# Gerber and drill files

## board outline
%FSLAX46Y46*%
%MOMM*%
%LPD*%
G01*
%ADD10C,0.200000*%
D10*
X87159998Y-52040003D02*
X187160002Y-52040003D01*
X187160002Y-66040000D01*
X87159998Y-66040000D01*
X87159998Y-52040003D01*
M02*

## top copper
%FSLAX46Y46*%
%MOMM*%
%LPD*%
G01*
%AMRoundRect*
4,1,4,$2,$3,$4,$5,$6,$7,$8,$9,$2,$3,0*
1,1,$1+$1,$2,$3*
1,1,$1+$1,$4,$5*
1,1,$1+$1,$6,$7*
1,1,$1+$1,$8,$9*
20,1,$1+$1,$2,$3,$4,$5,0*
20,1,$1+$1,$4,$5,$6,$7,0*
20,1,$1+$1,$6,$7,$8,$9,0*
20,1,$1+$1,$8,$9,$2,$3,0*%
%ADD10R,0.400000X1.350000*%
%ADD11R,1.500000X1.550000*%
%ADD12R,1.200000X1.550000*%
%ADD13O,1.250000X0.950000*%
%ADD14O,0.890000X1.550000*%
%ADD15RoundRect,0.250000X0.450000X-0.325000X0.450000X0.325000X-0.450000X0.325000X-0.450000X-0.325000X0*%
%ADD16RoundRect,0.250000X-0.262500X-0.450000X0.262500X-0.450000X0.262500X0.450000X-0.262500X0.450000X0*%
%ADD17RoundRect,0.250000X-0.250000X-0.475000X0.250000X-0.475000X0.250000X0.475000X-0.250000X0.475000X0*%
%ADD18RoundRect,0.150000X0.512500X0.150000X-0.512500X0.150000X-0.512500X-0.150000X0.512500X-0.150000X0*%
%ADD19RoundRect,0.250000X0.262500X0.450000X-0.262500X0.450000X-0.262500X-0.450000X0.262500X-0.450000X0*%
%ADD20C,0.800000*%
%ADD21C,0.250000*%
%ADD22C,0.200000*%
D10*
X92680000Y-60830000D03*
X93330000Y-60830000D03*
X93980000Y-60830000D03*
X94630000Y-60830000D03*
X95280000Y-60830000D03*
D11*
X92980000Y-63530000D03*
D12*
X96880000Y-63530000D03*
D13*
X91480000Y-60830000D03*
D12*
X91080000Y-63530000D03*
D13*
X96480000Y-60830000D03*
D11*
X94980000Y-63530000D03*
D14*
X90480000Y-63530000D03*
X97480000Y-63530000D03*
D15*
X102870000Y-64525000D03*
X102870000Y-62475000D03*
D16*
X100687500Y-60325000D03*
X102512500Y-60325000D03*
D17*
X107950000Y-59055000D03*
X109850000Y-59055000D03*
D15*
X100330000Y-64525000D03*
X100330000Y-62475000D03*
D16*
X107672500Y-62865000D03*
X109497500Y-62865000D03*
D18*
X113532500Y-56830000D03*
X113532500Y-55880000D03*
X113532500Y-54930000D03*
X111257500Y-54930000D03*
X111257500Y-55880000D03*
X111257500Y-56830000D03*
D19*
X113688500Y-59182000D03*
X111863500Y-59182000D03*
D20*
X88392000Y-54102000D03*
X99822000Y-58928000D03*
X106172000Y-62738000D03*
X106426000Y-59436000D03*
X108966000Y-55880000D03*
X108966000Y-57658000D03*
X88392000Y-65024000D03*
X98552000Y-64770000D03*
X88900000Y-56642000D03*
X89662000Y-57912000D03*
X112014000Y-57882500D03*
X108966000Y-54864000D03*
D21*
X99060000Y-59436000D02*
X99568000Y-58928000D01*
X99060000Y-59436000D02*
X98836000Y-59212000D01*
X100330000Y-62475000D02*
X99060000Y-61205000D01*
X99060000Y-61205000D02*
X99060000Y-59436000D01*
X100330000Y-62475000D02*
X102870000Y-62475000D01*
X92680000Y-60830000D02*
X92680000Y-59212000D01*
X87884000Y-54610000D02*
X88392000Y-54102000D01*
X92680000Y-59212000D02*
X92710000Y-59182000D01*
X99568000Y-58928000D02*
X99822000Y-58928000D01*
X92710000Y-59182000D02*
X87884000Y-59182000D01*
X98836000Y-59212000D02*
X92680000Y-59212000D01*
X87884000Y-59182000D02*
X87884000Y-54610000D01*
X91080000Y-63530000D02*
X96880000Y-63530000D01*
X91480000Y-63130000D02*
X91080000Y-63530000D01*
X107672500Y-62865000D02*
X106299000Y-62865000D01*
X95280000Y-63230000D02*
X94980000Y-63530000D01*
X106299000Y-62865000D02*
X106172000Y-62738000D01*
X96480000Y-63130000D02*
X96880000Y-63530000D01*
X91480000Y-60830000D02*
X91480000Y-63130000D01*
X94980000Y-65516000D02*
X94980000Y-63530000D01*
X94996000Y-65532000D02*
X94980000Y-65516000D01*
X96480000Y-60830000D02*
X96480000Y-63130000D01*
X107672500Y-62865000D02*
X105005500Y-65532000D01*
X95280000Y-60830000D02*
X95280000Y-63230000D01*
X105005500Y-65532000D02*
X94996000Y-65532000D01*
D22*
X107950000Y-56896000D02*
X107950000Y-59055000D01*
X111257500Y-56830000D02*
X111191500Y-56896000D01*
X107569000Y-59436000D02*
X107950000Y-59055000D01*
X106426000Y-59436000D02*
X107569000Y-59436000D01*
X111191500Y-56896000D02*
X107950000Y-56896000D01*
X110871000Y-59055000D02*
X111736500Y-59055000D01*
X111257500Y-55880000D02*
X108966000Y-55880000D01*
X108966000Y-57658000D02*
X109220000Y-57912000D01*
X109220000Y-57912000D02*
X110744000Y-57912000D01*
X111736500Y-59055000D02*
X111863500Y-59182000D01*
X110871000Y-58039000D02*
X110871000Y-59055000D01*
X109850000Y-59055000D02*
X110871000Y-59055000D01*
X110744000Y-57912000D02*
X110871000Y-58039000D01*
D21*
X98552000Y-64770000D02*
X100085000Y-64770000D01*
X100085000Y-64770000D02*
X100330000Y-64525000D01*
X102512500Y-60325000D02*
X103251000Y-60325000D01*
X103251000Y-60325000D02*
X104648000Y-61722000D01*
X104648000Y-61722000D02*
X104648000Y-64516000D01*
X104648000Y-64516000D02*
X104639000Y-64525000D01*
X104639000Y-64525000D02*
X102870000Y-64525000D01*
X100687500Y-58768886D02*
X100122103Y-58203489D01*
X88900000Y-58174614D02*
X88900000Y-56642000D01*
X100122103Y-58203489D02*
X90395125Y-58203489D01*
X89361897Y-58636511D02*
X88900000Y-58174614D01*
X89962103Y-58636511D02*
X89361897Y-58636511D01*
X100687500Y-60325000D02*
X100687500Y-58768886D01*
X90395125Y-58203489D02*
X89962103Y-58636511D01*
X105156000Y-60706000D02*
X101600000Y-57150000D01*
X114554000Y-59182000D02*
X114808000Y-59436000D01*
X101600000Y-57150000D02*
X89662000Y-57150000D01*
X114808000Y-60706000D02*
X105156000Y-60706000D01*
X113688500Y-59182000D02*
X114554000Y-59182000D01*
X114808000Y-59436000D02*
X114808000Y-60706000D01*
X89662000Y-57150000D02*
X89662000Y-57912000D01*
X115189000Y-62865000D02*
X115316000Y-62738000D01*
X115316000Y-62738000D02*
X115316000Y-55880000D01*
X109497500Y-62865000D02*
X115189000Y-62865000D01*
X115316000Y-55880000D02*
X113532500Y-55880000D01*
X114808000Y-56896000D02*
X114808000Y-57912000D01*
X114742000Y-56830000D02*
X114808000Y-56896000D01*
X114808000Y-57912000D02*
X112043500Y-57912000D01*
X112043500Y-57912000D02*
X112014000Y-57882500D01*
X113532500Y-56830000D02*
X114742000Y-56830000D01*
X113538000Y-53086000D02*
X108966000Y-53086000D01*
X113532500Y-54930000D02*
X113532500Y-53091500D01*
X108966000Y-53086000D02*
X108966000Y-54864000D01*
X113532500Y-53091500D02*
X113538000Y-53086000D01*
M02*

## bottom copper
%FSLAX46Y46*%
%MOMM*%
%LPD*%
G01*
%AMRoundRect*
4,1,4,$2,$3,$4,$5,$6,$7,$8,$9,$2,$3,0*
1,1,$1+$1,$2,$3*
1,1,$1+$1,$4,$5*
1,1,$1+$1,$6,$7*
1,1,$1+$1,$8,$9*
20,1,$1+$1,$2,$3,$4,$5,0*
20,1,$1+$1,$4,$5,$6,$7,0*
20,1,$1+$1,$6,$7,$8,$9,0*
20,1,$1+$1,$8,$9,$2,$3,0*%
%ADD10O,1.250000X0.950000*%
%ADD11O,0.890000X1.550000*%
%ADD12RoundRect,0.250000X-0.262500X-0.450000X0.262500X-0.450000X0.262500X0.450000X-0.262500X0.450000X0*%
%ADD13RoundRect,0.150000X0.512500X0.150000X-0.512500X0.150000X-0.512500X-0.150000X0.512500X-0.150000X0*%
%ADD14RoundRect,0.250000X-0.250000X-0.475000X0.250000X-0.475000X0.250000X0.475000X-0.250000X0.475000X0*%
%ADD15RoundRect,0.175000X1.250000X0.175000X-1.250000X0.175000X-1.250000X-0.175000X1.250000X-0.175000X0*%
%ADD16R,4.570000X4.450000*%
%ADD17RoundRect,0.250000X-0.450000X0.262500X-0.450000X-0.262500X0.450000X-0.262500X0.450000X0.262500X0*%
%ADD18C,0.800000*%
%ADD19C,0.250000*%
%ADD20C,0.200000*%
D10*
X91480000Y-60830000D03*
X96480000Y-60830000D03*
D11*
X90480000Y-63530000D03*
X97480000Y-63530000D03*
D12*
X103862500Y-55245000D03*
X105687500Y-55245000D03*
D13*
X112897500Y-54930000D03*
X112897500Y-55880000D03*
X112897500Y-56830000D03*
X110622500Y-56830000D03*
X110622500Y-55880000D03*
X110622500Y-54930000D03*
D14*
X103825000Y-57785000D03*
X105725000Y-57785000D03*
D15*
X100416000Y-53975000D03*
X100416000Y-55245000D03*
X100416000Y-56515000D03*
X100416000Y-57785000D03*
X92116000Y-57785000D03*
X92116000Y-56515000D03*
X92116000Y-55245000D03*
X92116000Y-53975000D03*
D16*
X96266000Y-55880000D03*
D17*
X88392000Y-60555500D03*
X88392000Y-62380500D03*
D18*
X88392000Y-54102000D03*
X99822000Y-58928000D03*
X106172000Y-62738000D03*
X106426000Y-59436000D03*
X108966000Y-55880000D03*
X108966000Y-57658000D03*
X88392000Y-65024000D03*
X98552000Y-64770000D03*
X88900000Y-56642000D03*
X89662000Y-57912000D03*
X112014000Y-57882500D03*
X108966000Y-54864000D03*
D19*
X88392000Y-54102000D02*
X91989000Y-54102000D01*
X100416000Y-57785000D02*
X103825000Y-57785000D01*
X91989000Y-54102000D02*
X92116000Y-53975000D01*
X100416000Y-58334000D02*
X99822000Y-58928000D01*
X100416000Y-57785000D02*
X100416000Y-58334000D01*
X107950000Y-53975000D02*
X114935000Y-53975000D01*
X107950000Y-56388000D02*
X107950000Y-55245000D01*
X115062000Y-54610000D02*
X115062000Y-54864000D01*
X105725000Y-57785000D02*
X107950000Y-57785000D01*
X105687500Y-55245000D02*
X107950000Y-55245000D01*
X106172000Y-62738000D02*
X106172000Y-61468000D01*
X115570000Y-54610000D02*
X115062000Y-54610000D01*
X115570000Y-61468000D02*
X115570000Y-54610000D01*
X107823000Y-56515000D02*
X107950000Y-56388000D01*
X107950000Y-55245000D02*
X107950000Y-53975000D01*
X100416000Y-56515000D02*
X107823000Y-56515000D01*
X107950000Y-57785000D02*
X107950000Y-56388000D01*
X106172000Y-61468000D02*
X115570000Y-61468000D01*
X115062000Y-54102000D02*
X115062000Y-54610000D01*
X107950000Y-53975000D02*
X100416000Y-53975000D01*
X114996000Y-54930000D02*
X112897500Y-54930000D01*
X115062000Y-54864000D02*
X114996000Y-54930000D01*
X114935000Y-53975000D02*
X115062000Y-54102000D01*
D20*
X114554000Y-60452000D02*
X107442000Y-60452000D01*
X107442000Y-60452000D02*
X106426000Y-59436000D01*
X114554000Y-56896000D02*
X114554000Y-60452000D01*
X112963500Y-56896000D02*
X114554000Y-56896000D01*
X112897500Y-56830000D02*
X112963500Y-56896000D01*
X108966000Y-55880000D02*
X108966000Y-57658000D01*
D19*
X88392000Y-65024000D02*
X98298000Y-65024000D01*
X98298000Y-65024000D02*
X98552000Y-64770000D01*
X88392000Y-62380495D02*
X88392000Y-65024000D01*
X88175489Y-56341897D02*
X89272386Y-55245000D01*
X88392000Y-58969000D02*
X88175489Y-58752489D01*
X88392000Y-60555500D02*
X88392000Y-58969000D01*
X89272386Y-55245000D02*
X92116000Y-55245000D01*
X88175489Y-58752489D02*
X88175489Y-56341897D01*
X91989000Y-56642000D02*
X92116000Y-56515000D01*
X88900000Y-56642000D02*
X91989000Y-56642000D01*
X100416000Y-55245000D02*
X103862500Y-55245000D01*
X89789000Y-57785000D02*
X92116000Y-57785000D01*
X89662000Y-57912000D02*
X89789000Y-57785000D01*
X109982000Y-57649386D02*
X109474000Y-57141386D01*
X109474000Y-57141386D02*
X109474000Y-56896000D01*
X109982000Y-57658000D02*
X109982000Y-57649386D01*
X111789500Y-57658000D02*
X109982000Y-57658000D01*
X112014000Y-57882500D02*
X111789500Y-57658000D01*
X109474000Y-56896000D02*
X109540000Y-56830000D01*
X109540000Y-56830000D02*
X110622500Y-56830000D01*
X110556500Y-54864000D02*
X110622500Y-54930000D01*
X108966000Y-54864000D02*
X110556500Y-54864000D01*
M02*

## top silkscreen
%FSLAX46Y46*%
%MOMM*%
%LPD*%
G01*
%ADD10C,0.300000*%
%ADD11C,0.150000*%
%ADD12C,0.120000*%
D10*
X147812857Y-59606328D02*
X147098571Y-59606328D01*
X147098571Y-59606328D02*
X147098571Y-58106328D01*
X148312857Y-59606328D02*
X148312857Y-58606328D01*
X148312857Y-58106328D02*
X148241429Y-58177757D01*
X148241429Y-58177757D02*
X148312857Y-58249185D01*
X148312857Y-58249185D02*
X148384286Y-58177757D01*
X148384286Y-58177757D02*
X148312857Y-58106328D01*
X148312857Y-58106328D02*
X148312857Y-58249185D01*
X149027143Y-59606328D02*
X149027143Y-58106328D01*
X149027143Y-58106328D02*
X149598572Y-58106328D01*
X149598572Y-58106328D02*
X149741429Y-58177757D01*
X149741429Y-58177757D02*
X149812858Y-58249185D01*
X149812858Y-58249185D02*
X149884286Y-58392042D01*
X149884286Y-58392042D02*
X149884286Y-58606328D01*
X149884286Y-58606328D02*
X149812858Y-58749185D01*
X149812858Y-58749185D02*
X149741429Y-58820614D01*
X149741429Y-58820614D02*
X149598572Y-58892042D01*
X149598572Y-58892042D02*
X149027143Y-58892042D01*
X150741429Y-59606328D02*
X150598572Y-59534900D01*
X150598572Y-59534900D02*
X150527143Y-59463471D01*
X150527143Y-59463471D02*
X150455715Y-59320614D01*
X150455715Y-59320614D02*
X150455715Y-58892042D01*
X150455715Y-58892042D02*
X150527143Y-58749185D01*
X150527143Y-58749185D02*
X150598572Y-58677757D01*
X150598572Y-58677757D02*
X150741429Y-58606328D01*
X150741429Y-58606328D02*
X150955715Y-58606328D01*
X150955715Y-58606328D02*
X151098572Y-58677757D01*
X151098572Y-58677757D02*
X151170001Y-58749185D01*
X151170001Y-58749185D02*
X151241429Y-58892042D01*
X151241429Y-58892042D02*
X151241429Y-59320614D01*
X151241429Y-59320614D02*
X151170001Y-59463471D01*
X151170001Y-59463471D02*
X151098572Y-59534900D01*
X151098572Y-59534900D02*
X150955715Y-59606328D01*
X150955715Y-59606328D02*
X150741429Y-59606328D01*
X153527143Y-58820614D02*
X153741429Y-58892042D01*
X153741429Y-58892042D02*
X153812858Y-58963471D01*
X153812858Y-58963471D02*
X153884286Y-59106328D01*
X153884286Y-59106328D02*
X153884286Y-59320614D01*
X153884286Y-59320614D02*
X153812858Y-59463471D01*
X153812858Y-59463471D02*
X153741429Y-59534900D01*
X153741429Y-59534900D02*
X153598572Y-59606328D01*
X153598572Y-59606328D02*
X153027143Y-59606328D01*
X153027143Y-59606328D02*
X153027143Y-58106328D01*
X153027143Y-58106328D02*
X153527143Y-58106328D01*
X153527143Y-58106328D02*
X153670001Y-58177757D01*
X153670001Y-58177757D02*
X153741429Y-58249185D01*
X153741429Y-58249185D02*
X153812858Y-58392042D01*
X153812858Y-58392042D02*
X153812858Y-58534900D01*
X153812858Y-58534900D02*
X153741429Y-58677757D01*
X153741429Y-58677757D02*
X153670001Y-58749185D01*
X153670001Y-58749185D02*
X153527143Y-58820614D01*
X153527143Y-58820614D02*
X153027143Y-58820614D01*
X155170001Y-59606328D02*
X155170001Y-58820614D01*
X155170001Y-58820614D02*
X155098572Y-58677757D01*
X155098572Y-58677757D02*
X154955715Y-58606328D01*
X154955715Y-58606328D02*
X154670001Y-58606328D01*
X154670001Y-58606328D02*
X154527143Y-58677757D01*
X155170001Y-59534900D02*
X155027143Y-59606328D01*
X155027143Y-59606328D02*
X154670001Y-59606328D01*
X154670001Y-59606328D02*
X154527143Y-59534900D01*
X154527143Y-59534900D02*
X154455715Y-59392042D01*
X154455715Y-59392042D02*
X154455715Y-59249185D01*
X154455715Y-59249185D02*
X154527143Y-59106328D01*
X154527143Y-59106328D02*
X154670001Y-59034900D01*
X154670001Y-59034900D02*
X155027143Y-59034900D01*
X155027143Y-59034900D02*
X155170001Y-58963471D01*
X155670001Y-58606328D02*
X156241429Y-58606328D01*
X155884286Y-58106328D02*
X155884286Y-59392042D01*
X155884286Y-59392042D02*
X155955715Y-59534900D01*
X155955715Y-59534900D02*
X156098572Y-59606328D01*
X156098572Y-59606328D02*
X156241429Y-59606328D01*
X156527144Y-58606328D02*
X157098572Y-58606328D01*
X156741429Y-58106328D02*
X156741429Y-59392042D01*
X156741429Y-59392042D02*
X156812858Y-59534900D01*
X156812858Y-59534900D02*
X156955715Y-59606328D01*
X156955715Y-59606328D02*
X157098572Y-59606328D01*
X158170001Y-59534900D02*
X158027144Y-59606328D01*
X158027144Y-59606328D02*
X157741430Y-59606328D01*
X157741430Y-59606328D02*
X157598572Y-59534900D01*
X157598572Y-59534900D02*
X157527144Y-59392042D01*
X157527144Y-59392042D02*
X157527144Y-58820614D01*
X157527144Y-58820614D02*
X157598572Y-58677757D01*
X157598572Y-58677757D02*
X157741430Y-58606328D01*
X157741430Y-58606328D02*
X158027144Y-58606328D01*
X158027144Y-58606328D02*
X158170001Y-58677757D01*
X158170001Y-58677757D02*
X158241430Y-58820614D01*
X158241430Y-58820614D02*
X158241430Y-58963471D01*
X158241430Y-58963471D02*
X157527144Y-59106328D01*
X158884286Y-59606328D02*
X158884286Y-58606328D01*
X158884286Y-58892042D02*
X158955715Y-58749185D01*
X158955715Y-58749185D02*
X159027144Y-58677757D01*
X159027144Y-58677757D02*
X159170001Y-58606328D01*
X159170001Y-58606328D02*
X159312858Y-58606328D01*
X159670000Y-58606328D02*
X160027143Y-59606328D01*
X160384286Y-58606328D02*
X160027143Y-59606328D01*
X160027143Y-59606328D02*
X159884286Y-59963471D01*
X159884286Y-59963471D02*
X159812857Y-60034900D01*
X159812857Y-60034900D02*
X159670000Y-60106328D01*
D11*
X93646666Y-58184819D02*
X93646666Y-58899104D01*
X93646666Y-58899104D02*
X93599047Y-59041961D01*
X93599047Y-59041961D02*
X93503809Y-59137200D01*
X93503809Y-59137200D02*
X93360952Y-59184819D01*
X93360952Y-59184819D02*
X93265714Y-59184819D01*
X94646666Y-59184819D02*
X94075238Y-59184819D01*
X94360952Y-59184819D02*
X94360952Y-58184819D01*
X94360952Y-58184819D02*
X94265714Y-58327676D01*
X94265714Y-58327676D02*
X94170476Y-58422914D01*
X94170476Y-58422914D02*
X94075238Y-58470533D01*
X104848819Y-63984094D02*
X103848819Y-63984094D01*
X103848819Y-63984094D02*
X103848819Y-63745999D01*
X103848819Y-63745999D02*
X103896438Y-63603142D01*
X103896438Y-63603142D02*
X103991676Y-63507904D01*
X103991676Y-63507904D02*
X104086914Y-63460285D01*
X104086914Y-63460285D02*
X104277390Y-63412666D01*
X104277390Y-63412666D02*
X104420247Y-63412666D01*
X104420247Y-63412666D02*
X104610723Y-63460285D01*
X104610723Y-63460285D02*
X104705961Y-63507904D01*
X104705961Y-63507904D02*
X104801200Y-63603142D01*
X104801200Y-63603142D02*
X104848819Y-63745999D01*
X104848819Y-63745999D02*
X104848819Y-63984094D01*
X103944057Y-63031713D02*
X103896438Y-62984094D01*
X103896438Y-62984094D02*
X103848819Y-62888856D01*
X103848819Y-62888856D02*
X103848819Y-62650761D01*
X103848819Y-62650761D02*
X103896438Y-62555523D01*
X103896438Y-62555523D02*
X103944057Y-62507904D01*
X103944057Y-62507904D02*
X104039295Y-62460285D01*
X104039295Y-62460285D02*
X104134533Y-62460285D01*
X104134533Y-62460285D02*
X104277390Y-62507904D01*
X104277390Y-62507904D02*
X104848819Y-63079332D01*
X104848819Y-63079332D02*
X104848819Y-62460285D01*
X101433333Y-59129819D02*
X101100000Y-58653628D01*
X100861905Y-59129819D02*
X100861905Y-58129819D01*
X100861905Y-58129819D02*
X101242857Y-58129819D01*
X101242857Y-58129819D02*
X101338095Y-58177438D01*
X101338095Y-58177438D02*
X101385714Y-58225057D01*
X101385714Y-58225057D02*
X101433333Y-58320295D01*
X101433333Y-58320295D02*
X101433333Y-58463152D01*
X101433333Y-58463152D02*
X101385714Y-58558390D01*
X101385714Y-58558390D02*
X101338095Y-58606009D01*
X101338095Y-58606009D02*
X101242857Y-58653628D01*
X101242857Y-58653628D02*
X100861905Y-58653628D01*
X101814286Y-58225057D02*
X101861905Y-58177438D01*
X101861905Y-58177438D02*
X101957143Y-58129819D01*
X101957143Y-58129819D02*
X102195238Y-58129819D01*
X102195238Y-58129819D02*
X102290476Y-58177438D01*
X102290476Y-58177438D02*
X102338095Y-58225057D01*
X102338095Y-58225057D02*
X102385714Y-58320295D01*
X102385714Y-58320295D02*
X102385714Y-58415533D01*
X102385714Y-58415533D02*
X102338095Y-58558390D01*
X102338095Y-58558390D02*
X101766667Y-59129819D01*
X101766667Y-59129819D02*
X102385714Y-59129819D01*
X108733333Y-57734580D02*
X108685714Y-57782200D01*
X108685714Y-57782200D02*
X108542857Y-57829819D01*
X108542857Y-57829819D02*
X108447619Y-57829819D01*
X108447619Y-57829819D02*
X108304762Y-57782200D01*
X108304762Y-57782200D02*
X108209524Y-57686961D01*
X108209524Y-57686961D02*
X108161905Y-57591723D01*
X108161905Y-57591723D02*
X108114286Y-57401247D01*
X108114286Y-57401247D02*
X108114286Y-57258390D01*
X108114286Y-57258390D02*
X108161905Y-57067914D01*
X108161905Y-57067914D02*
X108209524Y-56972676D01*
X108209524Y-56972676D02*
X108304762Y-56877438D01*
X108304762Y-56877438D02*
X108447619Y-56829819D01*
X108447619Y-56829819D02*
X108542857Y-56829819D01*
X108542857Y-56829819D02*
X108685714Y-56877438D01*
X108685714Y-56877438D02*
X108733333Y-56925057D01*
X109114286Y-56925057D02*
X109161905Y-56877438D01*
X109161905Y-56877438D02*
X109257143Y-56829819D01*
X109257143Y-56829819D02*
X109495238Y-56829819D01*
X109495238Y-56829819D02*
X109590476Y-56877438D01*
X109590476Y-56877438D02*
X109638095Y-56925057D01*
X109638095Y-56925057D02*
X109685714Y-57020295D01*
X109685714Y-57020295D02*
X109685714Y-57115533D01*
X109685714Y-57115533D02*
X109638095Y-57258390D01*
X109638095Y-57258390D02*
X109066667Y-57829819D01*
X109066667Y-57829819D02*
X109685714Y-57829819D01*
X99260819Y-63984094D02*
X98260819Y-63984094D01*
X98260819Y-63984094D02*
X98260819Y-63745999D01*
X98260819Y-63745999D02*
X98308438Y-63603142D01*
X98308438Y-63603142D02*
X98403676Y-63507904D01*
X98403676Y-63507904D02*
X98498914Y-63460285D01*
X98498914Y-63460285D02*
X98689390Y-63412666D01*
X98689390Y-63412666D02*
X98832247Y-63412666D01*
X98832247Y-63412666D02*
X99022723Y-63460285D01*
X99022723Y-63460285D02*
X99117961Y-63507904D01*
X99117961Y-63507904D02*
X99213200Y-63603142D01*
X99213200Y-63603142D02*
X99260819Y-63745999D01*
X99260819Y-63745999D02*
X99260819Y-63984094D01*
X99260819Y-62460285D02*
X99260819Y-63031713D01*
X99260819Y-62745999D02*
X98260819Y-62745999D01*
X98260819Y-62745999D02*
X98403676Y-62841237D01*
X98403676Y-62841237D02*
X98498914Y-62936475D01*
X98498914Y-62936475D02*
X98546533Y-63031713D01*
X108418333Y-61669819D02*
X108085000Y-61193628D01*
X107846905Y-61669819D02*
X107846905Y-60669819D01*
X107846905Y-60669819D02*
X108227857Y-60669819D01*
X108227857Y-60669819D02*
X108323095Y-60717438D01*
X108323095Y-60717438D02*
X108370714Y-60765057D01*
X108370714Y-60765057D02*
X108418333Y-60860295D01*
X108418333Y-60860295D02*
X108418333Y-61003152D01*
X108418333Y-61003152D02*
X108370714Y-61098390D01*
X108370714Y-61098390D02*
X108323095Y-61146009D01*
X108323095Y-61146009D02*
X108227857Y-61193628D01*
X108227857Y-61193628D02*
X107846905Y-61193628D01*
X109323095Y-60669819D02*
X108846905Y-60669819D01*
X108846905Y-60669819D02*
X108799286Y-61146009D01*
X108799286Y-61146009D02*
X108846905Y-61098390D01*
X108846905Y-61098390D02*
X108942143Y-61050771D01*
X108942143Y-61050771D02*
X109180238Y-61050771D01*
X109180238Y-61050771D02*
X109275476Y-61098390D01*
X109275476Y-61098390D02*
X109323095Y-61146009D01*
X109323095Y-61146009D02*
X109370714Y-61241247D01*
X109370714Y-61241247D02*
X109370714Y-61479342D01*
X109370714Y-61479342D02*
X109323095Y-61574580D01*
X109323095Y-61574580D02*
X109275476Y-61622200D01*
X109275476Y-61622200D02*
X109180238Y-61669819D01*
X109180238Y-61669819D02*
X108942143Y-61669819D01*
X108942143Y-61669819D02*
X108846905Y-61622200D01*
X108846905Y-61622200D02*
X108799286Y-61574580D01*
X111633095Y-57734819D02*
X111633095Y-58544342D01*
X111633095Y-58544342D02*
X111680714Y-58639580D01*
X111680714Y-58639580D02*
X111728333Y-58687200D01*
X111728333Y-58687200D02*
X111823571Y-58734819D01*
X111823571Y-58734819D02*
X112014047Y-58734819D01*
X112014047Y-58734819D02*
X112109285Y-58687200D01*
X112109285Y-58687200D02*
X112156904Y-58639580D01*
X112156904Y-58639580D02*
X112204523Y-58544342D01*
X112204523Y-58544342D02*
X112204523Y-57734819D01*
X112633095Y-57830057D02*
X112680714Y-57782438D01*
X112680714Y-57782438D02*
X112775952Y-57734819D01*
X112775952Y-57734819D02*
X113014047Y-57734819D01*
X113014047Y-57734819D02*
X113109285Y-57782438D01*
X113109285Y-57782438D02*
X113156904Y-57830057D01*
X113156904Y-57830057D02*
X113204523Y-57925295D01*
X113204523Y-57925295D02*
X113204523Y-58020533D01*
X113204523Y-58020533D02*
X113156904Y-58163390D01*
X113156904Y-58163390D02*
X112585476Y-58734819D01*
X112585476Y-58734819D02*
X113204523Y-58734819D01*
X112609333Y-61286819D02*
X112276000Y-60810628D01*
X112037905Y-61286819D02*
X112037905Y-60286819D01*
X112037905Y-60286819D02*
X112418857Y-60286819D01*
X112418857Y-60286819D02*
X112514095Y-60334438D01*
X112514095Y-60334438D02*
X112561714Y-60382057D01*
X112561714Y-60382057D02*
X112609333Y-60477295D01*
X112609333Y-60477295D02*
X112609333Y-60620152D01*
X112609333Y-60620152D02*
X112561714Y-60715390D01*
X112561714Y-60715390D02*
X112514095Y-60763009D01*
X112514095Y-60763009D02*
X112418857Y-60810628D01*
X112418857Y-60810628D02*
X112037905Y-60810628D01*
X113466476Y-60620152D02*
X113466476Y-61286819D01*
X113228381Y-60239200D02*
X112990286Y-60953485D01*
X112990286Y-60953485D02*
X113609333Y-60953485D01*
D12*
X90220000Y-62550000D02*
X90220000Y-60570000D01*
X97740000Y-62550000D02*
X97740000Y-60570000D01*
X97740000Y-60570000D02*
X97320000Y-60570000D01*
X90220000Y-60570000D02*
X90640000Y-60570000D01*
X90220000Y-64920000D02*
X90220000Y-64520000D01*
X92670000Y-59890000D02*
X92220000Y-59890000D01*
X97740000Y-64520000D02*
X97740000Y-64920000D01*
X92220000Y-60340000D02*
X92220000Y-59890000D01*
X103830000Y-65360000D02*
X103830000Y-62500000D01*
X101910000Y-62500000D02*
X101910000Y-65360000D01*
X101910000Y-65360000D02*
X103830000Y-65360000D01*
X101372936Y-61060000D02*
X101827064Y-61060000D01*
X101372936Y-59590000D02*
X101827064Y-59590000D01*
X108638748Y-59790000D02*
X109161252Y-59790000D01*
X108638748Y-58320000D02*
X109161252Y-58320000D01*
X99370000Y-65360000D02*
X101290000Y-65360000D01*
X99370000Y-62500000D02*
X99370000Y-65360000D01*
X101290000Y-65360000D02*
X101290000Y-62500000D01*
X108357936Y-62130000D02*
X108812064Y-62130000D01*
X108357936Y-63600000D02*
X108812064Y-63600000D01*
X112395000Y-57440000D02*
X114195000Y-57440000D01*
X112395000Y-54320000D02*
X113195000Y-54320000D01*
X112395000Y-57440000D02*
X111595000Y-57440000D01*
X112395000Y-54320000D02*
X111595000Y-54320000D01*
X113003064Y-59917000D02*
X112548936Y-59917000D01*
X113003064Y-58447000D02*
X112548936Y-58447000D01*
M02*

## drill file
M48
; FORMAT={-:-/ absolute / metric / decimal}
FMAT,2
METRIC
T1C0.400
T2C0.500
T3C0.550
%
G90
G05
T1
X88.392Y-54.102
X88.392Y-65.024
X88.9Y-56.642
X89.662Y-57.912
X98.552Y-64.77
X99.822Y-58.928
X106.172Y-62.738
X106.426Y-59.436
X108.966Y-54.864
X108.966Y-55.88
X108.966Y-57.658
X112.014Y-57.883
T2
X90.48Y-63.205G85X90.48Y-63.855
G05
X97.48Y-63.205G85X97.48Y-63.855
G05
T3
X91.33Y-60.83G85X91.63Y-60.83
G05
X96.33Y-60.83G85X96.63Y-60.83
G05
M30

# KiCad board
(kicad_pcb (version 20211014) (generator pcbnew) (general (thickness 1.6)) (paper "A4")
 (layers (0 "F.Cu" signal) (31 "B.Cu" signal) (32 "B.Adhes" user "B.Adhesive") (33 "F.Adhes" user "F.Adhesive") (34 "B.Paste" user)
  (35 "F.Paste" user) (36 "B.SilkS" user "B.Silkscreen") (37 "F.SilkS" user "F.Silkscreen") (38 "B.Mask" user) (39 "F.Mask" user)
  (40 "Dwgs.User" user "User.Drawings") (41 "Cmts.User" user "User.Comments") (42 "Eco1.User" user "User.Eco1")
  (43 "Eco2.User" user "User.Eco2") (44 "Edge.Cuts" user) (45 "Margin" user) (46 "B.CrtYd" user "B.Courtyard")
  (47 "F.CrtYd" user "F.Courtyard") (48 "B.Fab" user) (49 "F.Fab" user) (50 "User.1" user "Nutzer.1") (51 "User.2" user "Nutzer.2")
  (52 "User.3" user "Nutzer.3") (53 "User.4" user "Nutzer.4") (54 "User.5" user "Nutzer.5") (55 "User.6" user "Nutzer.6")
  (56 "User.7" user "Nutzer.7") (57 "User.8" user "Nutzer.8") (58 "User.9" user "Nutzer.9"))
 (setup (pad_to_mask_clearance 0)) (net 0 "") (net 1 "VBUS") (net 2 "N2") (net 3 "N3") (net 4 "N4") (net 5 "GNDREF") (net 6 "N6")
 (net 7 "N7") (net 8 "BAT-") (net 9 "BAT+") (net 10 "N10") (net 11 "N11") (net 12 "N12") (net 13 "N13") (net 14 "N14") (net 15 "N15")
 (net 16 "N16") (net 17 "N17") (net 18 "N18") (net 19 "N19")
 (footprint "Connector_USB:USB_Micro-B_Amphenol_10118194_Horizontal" (layer "F.Cu") (at 93.98 62.23)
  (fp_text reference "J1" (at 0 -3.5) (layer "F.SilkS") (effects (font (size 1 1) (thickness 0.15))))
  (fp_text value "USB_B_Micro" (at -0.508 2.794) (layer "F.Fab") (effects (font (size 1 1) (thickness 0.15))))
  (fp_line (start -3.76 0.32) (end -3.76 -1.66) (layer "F.SilkS") (width 0.12))
  (fp_line (start 3.76 0.32) (end 3.76 -1.66) (layer "F.SilkS") (width 0.12))
  (fp_line (start 3.76 -1.66) (end 3.34 -1.66) (layer "F.SilkS") (width 0.12))
  (fp_line (start -3.76 -1.66) (end -3.34 -1.66) (layer "F.SilkS") (width 0.12))
  (fp_line (start -3.76 2.69) (end -3.76 2.29) (layer "F.SilkS") (width 0.12))
  (fp_line (start -1.31 -2.34) (end -1.76 -2.34) (layer "F.SilkS") (width 0.12))
  (fp_line (start 3.76 2.29) (end 3.76 2.69) (layer "F.SilkS") (width 0.12))
  (fp_line (start -1.76 -1.89) (end -1.76 -2.34) (layer "F.SilkS") (width 0.12))
  (pad "" smd oval locked (at 2.5 -1.4) (size 1.25 0.95) (layers "F.Paste"))
  (pad "" smd oval locked (at -3.5 1.3) (size 0.89 1.55) (layers "F.Paste"))
  (pad "" smd oval locked (at -2.5 -1.4) (size 1.25 0.95) (layers "F.Paste"))
  (pad "" smd oval locked (at 3.5 1.3) (size 0.89 1.55) (layers "F.Paste"))
  (pad "1" smd rect locked (at -1.3 -1.4) (size 0.4 1.35) (layers "F.Cu" "F.Paste" "F.Mask") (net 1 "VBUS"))
  (pad "2" smd rect locked (at -0.65 -1.4) (size 0.4 1.35) (layers "F.Cu" "F.Paste" "F.Mask") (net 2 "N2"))
  (pad "3" smd rect locked (at 0 -1.4) (size 0.4 1.35) (layers "F.Cu" "F.Paste" "F.Mask") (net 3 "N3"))
  (pad "4" smd rect locked (at 0.65 -1.4) (size 0.4 1.35) (layers "F.Cu" "F.Paste" "F.Mask") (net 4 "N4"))
  (pad "5" smd rect locked (at 1.3 -1.4) (size 0.4 1.35) (layers "F.Cu" "F.Paste" "F.Mask") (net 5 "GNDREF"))
  (pad "6" smd rect locked (at -1 1.3) (size 1.5 1.55) (layers "F.Cu" "F.Paste" "F.Mask") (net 5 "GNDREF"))
  (pad "6" smd rect locked (at 2.9 1.3) (size 1.2 1.55) (layers "F.Cu" "F.Paste" "F.Mask") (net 5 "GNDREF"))
  (pad "6" thru_hole oval locked (at -2.5 -1.4) (size 1.25 0.95) (drill oval 0.85 0.55) (layers *.Cu *.Mask) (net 5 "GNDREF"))
  (pad "6" smd rect locked (at -2.9 1.3) (size 1.2 1.55) (layers "F.Cu" "F.Paste" "F.Mask") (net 5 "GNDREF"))
  (pad "6" thru_hole oval locked (at 2.5 -1.4) (size 1.25 0.95) (drill oval 0.85 0.55) (layers *.Cu *.Mask) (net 5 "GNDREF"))
  (pad "6" smd rect locked (at 1 1.3) (size 1.5 1.55) (layers "F.Cu" "F.Paste" "F.Mask") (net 5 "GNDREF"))
  (pad "6" thru_hole oval locked (at -3.5 1.3) (size 0.89 1.55) (drill oval 0.5 1.15) (layers *.Cu *.Mask) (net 5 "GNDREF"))
  (pad "6" thru_hole oval locked (at 3.5 1.3) (size 0.89 1.55) (drill oval 0.5 1.15) (layers *.Cu *.Mask) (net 5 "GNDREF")))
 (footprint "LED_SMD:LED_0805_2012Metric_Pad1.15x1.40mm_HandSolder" (layer "F.Cu") (at 102.87 63.5 90)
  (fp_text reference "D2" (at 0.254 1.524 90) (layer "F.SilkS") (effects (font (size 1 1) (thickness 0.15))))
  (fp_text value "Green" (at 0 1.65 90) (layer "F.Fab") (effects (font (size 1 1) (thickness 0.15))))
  (fp_line (start -1.86 0.96) (end 1 0.96) (layer "F.SilkS") (width 0.12))
  (fp_line (start 1 -0.96) (end -1.86 -0.96) (layer "F.SilkS") (width 0.12))
  (fp_line (start -1.86 -0.96) (end -1.86 0.96) (layer "F.SilkS") (width 0.12))
  (pad "1" smd roundrect locked (at -1.025 0 90) (size 1.15 1.4) (layers "F.Cu" "F.Paste" "F.Mask") (roundrect_rratio 0.217391) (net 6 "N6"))
  (pad "2" smd roundrect locked (at 1.025 0 90) (size 1.15 1.4) (layers "F.Cu" "F.Paste" "F.Mask") (roundrect_rratio 0.217391)
   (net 1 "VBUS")))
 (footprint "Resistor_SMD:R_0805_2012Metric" (layer "F.Cu") (at 101.6 60.325)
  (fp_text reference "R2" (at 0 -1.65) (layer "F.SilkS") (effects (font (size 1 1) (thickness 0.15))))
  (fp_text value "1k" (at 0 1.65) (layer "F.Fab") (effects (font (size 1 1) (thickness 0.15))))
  (fp_line (start -0.227064 0.735) (end 0.227064 0.735) (layer "F.SilkS") (width 0.12))
  (fp_line (start -0.227064 -0.735) (end 0.227064 -0.735) (layer "F.SilkS") (width 0.12))
  (pad "1" smd roundrect locked (at -0.9125 0) (size 1.025 1.4) (layers "F.Cu" "F.Paste" "F.Mask") (roundrect_rratio 0.243902) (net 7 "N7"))
  (pad "2" smd roundrect locked (at 0.9125 0) (size 1.025 1.4) (layers "F.Cu" "F.Paste" "F.Mask") (roundrect_rratio 0.243902) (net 6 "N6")))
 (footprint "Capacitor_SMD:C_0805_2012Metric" (layer "F.Cu") (at 108.9 59.055) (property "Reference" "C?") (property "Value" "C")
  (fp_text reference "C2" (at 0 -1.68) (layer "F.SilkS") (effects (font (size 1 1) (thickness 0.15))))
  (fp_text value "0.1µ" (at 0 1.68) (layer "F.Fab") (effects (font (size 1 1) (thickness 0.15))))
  (fp_line (start -0.261252 0.735) (end 0.261252 0.735) (layer "F.SilkS") (width 0.12))
  (fp_line (start -0.261252 -0.735) (end 0.261252 -0.735) (layer "F.SilkS") (width 0.12))
  (pad "1" smd roundrect locked (at -0.95 0) (size 1 1.45) (layers "F.Cu" "F.Paste" "F.Mask") (roundrect_rratio 0.25) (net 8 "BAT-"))
  (pad "2" smd roundrect locked (at 0.95 0) (size 1 1.45) (layers "F.Cu" "F.Paste" "F.Mask") (roundrect_rratio 0.25) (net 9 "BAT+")))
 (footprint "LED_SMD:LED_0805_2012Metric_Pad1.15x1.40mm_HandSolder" (layer "F.Cu") (at 100.33 63.5 90) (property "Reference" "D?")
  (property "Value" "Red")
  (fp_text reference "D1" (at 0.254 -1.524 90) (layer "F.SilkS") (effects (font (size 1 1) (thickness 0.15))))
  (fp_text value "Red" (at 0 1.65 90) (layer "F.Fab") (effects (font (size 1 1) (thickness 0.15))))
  (fp_line (start -1.86 -0.96) (end -1.86 0.96) (layer "F.SilkS") (width 0.12))
  (fp_line (start 1 -0.96) (end -1.86 -0.96) (layer "F.SilkS") (width 0.12))
  (fp_line (start -1.86 0.96) (end 1 0.96) (layer "F.SilkS") (width 0.12))
  (pad "1" smd roundrect locked (at -1.025 0 90) (size 1.15 1.4) (layers "F.Cu" "F.Paste" "F.Mask") (roundrect_rratio 0.217391)
   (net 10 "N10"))
  (pad "2" smd roundrect locked (at 1.025 0 90) (size 1.15 1.4) (layers "F.Cu" "F.Paste" "F.Mask") (roundrect_rratio 0.217391)
   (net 1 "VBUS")))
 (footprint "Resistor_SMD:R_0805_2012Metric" (layer "F.Cu") (at 108.585 62.865)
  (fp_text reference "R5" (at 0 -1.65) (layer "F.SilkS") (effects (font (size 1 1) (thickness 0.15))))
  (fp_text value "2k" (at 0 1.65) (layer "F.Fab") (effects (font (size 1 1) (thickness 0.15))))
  (fp_line (start -0.227064 -0.735) (end 0.227064 -0.735) (layer "F.SilkS") (width 0.12))
  (fp_line (start -0.227064 0.735) (end 0.227064 0.735) (layer "F.SilkS") (width 0.12))
  (pad "1" smd roundrect locked (at -0.9125 0) (size 1.025 1.4) (layers "F.Cu" "F.Paste" "F.Mask") (roundrect_rratio 0.243902)
   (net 5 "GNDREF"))
  (pad "2" smd roundrect locked (at 0.9125 0) (size 1.025 1.4) (layers "F.Cu" "F.Paste" "F.Mask") (roundrect_rratio 0.243902) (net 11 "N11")))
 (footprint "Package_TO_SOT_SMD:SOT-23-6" (layer "F.Cu") (at 112.395 55.88 180) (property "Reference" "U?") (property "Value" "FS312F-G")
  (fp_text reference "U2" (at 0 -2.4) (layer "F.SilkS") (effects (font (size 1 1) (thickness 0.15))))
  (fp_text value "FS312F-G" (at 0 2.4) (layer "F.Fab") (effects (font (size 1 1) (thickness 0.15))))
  (fp_line (start 0 -1.56) (end -1.8 -1.56) (layer "F.SilkS") (width 0.12))
  (fp_line (start 0 1.56) (end -0.8 1.56) (layer "F.SilkS") (width 0.12))
  (fp_line (start 0 -1.56) (end 0.8 -1.56) (layer "F.SilkS") (width 0.12))
  (fp_line (start 0 1.56) (end 0.8 1.56) (layer "F.SilkS") (width 0.12))
  (pad "1" smd roundrect locked (at -1.1375 -0.95 180) (size 1.325 0.6) (layers "F.Cu" "F.Paste" "F.Mask") (roundrect_rratio 0.25)
   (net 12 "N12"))
  (pad "2" smd roundrect locked (at -1.1375 0 180) (size 1.325 0.6) (layers "F.Cu" "F.Paste" "F.Mask") (roundrect_rratio 0.25)
   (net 11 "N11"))
  (pad "3" smd roundrect locked (at -1.1375 0.95 180) (size 1.325 0.6) (layers "F.Cu" "F.Paste" "F.Mask") (roundrect_rratio 0.25)
   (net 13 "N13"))
  (pad "4" smd roundrect locked (at 1.1375 0.95 180) (size 1.325 0.6) (layers "F.Cu" "F.Paste" "F.Mask") (roundrect_rratio 0.25)
   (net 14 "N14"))
  (pad "5" smd roundrect locked (at 1.1375 0 180) (size 1.325 0.6) (layers "F.Cu" "F.Paste" "F.Mask") (roundrect_rratio 0.25) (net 9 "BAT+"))
  (pad "6" smd roundrect locked (at 1.1375 -0.95 180) (size 1.325 0.6) (layers "F.Cu" "F.Paste" "F.Mask") (roundrect_rratio 0.25)
   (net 8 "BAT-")))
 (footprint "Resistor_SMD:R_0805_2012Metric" (layer "F.Cu") (at 112.776 59.182 180)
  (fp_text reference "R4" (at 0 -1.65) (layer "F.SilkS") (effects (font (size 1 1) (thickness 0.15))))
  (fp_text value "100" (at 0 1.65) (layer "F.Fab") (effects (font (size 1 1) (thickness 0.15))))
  (fp_line (start -0.227064 -0.735) (end 0.227064 -0.735) (layer "F.SilkS") (width 0.12))
  (fp_line (start -0.227064 0.735) (end 0.227064 0.735) (layer "F.SilkS") (width 0.12))
  (pad "1" smd roundrect locked (at -0.9125 0 180) (size 1.025 1.4) (layers "F.Cu" "F.Paste" "F.Mask") (roundrect_rratio 0.243902)
   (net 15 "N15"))
  (pad "2" smd roundrect locked (at 0.9125 0 180) (size 1.025 1.4) (layers "F.Cu" "F.Paste" "F.Mask") (roundrect_rratio 0.243902)
   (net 9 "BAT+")))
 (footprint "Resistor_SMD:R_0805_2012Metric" (layer "B.Cu") (at 104.775 55.245)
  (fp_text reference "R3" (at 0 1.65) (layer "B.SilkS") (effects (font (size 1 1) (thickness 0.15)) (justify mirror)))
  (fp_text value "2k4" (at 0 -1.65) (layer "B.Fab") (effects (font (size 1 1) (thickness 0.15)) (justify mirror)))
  (pad "1" smd roundrect locked (at -0.9125 0) (size 1.025 1.4) (layers "B.Cu" "B.Paste" "B.Mask") (roundrect_rratio 0.243902)
   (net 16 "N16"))
  (pad "2" smd roundrect locked (at 0.9125 0) (size 1.025 1.4) (layers "B.Cu" "B.Paste" "B.Mask") (roundrect_rratio 0.243902)
   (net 5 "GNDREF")))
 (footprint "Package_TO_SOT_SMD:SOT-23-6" (layer "B.Cu") (at 111.76 55.88 180) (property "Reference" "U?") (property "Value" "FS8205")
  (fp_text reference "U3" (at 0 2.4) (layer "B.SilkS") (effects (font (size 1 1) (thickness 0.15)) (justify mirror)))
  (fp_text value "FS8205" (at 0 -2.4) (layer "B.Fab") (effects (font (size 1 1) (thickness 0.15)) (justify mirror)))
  (pad "1" smd roundrect locked (at -1.1375 0.95 180) (size 1.325 0.6) (layers "B.Cu" "B.Paste" "B.Mask") (roundrect_rratio 0.25)
   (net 5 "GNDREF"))
  (pad "2" smd roundrect locked (at -1.1375 0 180) (size 1.325 0.6) (layers "B.Cu" "B.Paste" "B.Mask") (roundrect_rratio 0.25)
   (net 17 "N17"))
  (pad "3" smd roundrect locked (at -1.1375 -0.95 180) (size 1.325 0.6) (layers "B.Cu" "B.Paste" "B.Mask") (roundrect_rratio 0.25)
   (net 8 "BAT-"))
  (pad "4" smd roundrect locked (at 1.1375 -0.95 180) (size 1.325 0.6) (layers "B.Cu" "B.Paste" "B.Mask") (roundrect_rratio 0.25)
   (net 12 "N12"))
  (pad "5" smd roundrect locked (at 1.1375 0 180) (size 1.325 0.6) (layers "B.Cu" "B.Paste" "B.Mask") (roundrect_rratio 0.25) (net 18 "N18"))
  (pad "6" smd roundrect locked (at 1.1375 0.95 180) (size 1.325 0.6) (layers "B.Cu" "B.Paste" "B.Mask") (roundrect_rratio 0.25)
   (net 13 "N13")))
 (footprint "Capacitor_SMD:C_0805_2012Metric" (layer "B.Cu") (at 104.775 57.785) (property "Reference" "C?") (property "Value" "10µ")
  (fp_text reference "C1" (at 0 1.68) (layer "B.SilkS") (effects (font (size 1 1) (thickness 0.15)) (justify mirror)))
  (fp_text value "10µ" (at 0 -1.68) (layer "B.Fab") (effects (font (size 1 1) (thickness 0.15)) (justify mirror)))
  (pad "1" smd roundrect locked (at -0.95 0) (size 1 1.45) (layers "B.Cu" "B.Paste" "B.Mask") (roundrect_rratio 0.25) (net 1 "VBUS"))
  (pad "2" smd roundrect locked (at 0.95 0) (size 1 1.45) (layers "B.Cu" "B.Paste" "B.Mask") (roundrect_rratio 0.25) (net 5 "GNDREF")))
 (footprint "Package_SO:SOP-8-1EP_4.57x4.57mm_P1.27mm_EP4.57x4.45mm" (layer "B.Cu") (at 96.266 55.88 180) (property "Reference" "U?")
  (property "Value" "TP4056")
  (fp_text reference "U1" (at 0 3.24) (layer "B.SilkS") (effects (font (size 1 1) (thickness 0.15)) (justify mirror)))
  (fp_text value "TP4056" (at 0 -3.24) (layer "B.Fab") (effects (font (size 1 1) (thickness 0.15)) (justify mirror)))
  (pad "" smd roundrect locked (at -1.14 1.11 180) (size 1.84 1.79) (layers "B.Paste") (roundrect_rratio 0.139665))
  (pad "" smd roundrect locked (at -1.14 -1.11 180) (size 1.84 1.79) (layers "B.Paste") (roundrect_rratio 0.139665))
  (pad "" smd roundrect locked (at 1.14 1.11 180) (size 1.84 1.79) (layers "B.Paste") (roundrect_rratio 0.139665))
  (pad "" smd roundrect locked (at 1.14 -1.11 180) (size 1.84 1.79) (layers "B.Paste") (roundrect_rratio 0.139665))
  (pad "1" smd roundrect locked (at -4.15 1.905 180) (size 2.85 0.7) (layers "B.Cu" "B.Paste" "B.Mask") (roundrect_rratio 0.25)
   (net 5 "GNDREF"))
  (pad "2" smd roundrect locked (at -4.15 0.635 180) (size 2.85 0.7) (layers "B.Cu" "B.Paste" "B.Mask") (roundrect_rratio 0.25)
   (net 16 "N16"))
  (pad "3" smd roundrect locked (at -4.15 -0.635 180) (size 2.85 0.7) (layers "B.Cu" "B.Paste" "B.Mask") (roundrect_rratio 0.25)
   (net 5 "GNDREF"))
  (pad "4" smd roundrect locked (at -4.15 -1.905 180) (size 2.85 0.7) (layers "B.Cu" "B.Paste" "B.Mask") (roundrect_rratio 0.25)
   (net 1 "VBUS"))
  (pad "5" smd roundrect locked (at 4.15 -1.905 180) (size 2.85 0.7) (layers "B.Cu" "B.Paste" "B.Mask") (roundrect_rratio 0.25)
   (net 15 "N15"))
  (pad "6" smd roundrect locked (at 4.15 -0.635 180) (size 2.85 0.7) (layers "B.Cu" "B.Paste" "B.Mask") (roundrect_rratio 0.25) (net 7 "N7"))
  (pad "7" smd roundrect locked (at 4.15 0.635 180) (size 2.85 0.7) (layers "B.Cu" "B.Paste" "B.Mask") (roundrect_rratio 0.25)
   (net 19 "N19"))
  (pad "8" smd roundrect locked (at 4.15 1.905 180) (size 2.85 0.7) (layers "B.Cu" "B.Paste" "B.Mask") (roundrect_rratio 0.25)
   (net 1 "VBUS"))
  (pad "9" smd rect locked (at 0 0 180) (size 4.57 4.45) (layers "B.Cu" "B.Mask")))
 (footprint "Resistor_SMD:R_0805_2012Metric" (layer "B.Cu") (at 88.392 61.468 -90) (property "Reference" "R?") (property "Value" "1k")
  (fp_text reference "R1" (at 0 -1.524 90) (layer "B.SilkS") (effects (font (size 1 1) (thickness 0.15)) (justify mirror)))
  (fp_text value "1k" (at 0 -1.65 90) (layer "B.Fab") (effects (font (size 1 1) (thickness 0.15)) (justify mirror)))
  (pad "1" smd roundrect locked (at -0.9125 0 270) (size 1.025 1.4) (layers "B.Cu" "B.Paste" "B.Mask") (roundrect_rratio 0.243902)
   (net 19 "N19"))
  (pad "2" smd roundrect locked (at 0.9125 0 270) (size 1.025 1.4) (layers "B.Cu" "B.Paste" "B.Mask") (roundrect_rratio 0.243902)
   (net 10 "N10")))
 (gr_rect (start 87.159998 52.040003) (end 187.160002 66.04) (layer "Edge.Cuts") (width 0.2) (fill none))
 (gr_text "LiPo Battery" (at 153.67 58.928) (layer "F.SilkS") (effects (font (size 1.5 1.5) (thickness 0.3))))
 (segment (start 99.06 59.436) (end 99.568 58.928) (width 0.25) (layer "F.Cu") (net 1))
 (segment (start 99.06 59.436) (end 98.836 59.212) (width 0.25) (layer "F.Cu") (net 1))
 (segment (start 100.33 62.475) (end 99.06 61.205) (width 0.25) (layer "F.Cu") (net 1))
 (segment (start 99.06 61.205) (end 99.06 59.436) (width 0.25) (layer "F.Cu") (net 1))
 (segment (start 100.33 62.475) (end 102.87 62.475) (width 0.25) (layer "F.Cu") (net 1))
 (segment (start 92.68 60.83) (end 92.68 59.212) (width 0.25) (layer "F.Cu") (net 1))
 (segment (start 87.884 54.61) (end 88.392 54.102) (width 0.25) (layer "F.Cu") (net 1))
 (segment (start 92.68 59.212) (end 92.71 59.182) (width 0.25) (layer "F.Cu") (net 1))
 (segment (start 99.568 58.928) (end 99.822 58.928) (width 0.25) (layer "F.Cu") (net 1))
 (segment (start 92.71 59.182) (end 87.884 59.182) (width 0.25) (layer "F.Cu") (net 1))
 (segment (start 98.836 59.212) (end 92.68 59.212) (width 0.25) (layer "F.Cu") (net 1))
 (segment (start 87.884 59.182) (end 87.884 54.61) (width 0.25) (layer "F.Cu") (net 1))
 (via (at 88.392 54.102) (size 0.8) (drill 0.4) (layers "F.Cu" "B.Cu") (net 1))
 (via (at 99.822 58.928) (size 0.8) (drill 0.4) (layers "F.Cu" "B.Cu") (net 1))
 (segment (start 88.392 54.102) (end 91.989 54.102) (width 0.25) (layer "B.Cu") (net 1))
 (segment (start 100.416 57.785) (end 103.825 57.785) (width 0.25) (layer "B.Cu") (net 1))
 (segment (start 91.989 54.102) (end 92.116 53.975) (width 0.25) (layer "B.Cu") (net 1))
 (segment (start 100.416 58.334) (end 99.822 58.928) (width 0.25) (layer "B.Cu") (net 1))
 (segment (start 100.416 57.785) (end 100.416 58.334) (width 0.25) (layer "B.Cu") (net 1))
 (segment (start 91.08 63.53) (end 96.88 63.53) (width 0.25) (layer "F.Cu") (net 5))
 (segment (start 91.48 63.13) (end 91.08 63.53) (width 0.25) (layer "F.Cu") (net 5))
 (segment (start 107.6725 62.865) (end 106.299 62.865) (width 0.25) (layer "F.Cu") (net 5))
 (segment (start 95.28 63.23) (end 94.98 63.53) (width 0.25) (layer "F.Cu") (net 5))
 (segment (start 106.299 62.865) (end 106.172 62.738) (width 0.25) (layer "F.Cu") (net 5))
 (segment (start 96.48 63.13) (end 96.88 63.53) (width 0.25) (layer "F.Cu") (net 5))
 (segment (start 91.48 60.83) (end 91.48 63.13) (width 0.25) (layer "F.Cu") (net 5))
 (segment (start 94.98 65.516) (end 94.98 63.53) (width 0.25) (layer "F.Cu") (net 5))
 (segment (start 94.996 65.532) (end 94.98 65.516) (width 0.25) (layer "F.Cu") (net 5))
 (segment (start 96.48 60.83) (end 96.48 63.13) (width 0.25) (layer "F.Cu") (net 5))
 (segment (start 107.6725 62.865) (end 105.0055 65.532) (width 0.25) (layer "F.Cu") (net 5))
 (segment (start 95.28 60.83) (end 95.28 63.23) (width 0.25) (layer "F.Cu") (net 5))
 (segment (start 105.0055 65.532) (end 94.996 65.532) (width 0.25) (layer "F.Cu") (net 5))
 (via (at 106.172 62.738) (size 0.8) (drill 0.4) (layers "F.Cu" "B.Cu") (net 5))
 (segment (start 107.95 53.975) (end 114.935 53.975) (width 0.25) (layer "B.Cu") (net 5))
 (segment (start 107.95 56.388) (end 107.95 55.245) (width 0.25) (layer "B.Cu") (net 5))
 (segment (start 115.062 54.61) (end 115.062 54.864) (width 0.25) (layer "B.Cu") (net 5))
 (segment (start 105.725 57.785) (end 107.95 57.785) (width 0.25) (layer "B.Cu") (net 5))
 (segment (start 105.6875 55.245) (end 107.95 55.245) (width 0.25) (layer "B.Cu") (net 5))
 (segment (start 106.172 62.738) (end 106.172 61.468) (width 0.25) (layer "B.Cu") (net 5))
 (segment (start 115.57 54.61) (end 115.062 54.61) (width 0.25) (layer "B.Cu") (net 5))
 (segment (start 115.57 61.468) (end 115.57 54.61) (width 0.25) (layer "B.Cu") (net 5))
 (segment (start 107.823 56.515) (end 107.95 56.388) (width 0.25) (layer "B.Cu") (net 5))
 (segment (start 107.95 55.245) (end 107.95 53.975) (width 0.25) (layer "B.Cu") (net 5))
 (segment (start 100.416 56.515) (end 107.823 56.515) (width 0.25) (layer "B.Cu") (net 5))
 (segment (start 107.95 57.785) (end 107.95 56.388) (width 0.25) (layer "B.Cu") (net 5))
 (segment (start 106.172 61.468) (end 115.57 61.468) (width 0.25) (layer "B.Cu") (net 5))
 (segment (start 115.062 54.102) (end 115.062 54.61) (width 0.25) (layer "B.Cu") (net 5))
 (segment (start 107.95 53.975) (end 100.416 53.975) (width 0.25) (layer "B.Cu") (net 5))
 (segment (start 114.996 54.93) (end 112.8975 54.93) (width 0.25) (layer "B.Cu") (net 5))
 (segment (start 115.062 54.864) (end 114.996 54.93) (width 0.25) (layer "B.Cu") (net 5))
 (segment (start 114.935 53.975) (end 115.062 54.102) (width 0.25) (layer "B.Cu") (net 5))
 (segment (start 107.95 56.896) (end 107.95 59.055) (width 0.2) (layer "F.Cu") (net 8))
 (segment (start 111.2575 56.83) (end 111.1915 56.896) (width 0.2) (layer "F.Cu") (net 8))
 (segment (start 107.569 59.436) (end 107.95 59.055) (width 0.2) (layer "F.Cu") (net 8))
 (segment (start 106.426 59.436) (end 107.569 59.436) (width 0.2) (layer "F.Cu") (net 8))
 (segment (start 111.1915 56.896) (end 107.95 56.896) (width 0.2) (layer "F.Cu") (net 8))
 (via (at 106.426 59.436) (size 0.8) (drill 0.4) (layers "F.Cu" "B.Cu") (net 8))
 (segment (start 114.554 60.452) (end 107.442 60.452) (width 0.2) (layer "B.Cu") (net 8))
 (segment (start 107.442 60.452) (end 106.426 59.436) (width 0.2) (layer "B.Cu") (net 8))
 (segment (start 114.554 56.896) (end 114.554 60.452) (width 0.2) (layer "B.Cu") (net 8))
 (segment (start 112.9635 56.896) (end 114.554 56.896) (width 0.2) (layer "B.Cu") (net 8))
 (segment (start 112.8975 56.83) (end 112.9635 56.896) (width 0.2) (layer "B.Cu") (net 8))
 (segment (start 110.871 59.055) (end 111.7365 59.055) (width 0.2) (layer "F.Cu") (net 9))
 (segment (start 111.2575 55.88) (end 108.966 55.88) (width 0.2) (layer "F.Cu") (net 9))
 (segment (start 108.966 57.658) (end 109.22 57.912) (width 0.2) (layer "F.Cu") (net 9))
 (segment (start 109.22 57.912) (end 110.744 57.912) (width 0.2) (layer "F.Cu") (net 9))
 (segment (start 111.7365 59.055) (end 111.8635 59.182) (width 0.2) (layer "F.Cu") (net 9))
 (segment (start 110.871 58.039) (end 110.871 59.055) (width 0.2) (layer "F.Cu") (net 9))
 (segment (start 109.85 59.055) (end 110.871 59.055) (width 0.2) (layer "F.Cu") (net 9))
 (segment (start 110.744 57.912) (end 110.871 58.039) (width 0.2) (layer "F.Cu") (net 9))
 (via (at 108.966 55.88) (size 0.8) (drill 0.4) (layers "F.Cu" "B.Cu") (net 9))
 (via (at 108.966 57.658) (size 0.8) (drill 0.4) (layers "F.Cu" "B.Cu") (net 9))
 (segment (start 108.966 55.88) (end 108.966 57.658) (width 0.2) (layer "B.Cu") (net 9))
 (segment (start 98.552 64.77) (end 100.085 64.77) (width 0.25) (layer "F.Cu") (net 10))
 (segment (start 100.085 64.77) (end 100.33 64.525) (width 0.25) (layer "F.Cu") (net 10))
 (via (at 88.392 65.024) (size 0.8) (drill 0.4) (layers "F.Cu" "B.Cu") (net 10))
 (via (at 98.552 64.77) (size 0.8) (drill 0.4) (layers "F.Cu" "B.Cu") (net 10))
 (segment (start 88.392 65.024) (end 98.298 65.024) (width 0.25) (layer "B.Cu") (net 10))
 (segment (start 98.298 65.024) (end 98.552 64.77) (width 0.25) (layer "B.Cu") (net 10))
 (segment (start 88.392 62.380495) (end 88.392 65.024) (width 0.25) (layer "B.Cu") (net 10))
 (segment (start 102.5125 60.325) (end 103.251 60.325) (width 0.25) (layer "F.Cu") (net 6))
 (segment (start 103.251 60.325) (end 104.648 61.722) (width 0.25) (layer "F.Cu") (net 6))
 (segment (start 104.648 61.722) (end 104.648 64.516) (width 0.25) (layer "F.Cu") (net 6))
 (segment (start 104.648 64.516) (end 104.639 64.525) (width 0.25) (layer "F.Cu") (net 6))
 (segment (start 104.639 64.525) (end 102.87 64.525) (width 0.25) (layer "F.Cu") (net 6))
 (segment (start 88.175489 56.341897) (end 89.272386 55.245) (width 0.25) (layer "B.Cu") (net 19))
 (segment (start 88.392 58.969) (end 88.175489 58.752489) (width 0.25) (layer "B.Cu") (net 19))
 (segment (start 88.392 60.5555) (end 88.392 58.969) (width 0.25) (layer "B.Cu") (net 19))
 (segment (start 89.272386 55.245) (end 92.116 55.245) (width 0.25) (layer "B.Cu") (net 19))
 (segment (start 88.175489 58.752489) (end 88.175489 56.341897) (width 0.25) (layer "B.Cu") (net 19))
 (segment (start 100.6875 58.768886) (end 100.122103 58.203489) (width 0.25) (layer "F.Cu") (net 7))
 (segment (start 88.9 58.174614) (end 88.9 56.642) (width 0.25) (layer "F.Cu") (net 7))
 (segment (start 100.122103 58.203489) (end 90.395125 58.203489) (width 0.25) (layer "F.Cu") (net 7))
 (segment (start 89.361897 58.636511) (end 88.9 58.174614) (width 0.25) (layer "F.Cu") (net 7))
 (segment (start 89.962103 58.636511) (end 89.361897 58.636511) (width 0.25) (layer "F.Cu") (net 7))
 (segment (start 100.6875 60.325) (end 100.6875 58.768886) (width 0.25) (layer "F.Cu") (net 7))
 (segment (start 90.395125 58.203489) (end 89.962103 58.636511) (width 0.25) (layer "F.Cu") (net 7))
 (via (at 88.9 56.642) (size 0.8) (drill 0.4) (layers "F.Cu" "B.Cu") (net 7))
 (segment (start 91.989 56.642) (end 92.116 56.515) (width 0.25) (layer "B.Cu") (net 7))
 (segment (start 88.9 56.642) (end 91.989 56.642) (width 0.25) (layer "B.Cu") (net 7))
 (segment (start 100.416 55.245) (end 103.8625 55.245) (width 0.25) (layer "B.Cu") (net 16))
 (segment (start 105.156 60.706) (end 101.6 57.15) (width 0.25) (layer "F.Cu") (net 15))
 (segment (start 114.554 59.182) (end 114.808 59.436) (width 0.25) (layer "F.Cu") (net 15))
 (segment (start 101.6 57.15) (end 89.662 57.15) (width 0.25) (layer "F.Cu") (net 15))
 (segment (start 114.808 60.706) (end 105.156 60.706) (width 0.25) (layer "F.Cu") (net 15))
 (segment (start 113.6885 59.182) (end 114.554 59.182) (width 0.25) (layer "F.Cu") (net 15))
 (segment (start 114.808 59.436) (end 114.808 60.706) (width 0.25) (layer "F.Cu") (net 15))
 (segment (start 89.662 57.15) (end 89.662 57.912) (width 0.25) (layer "F.Cu") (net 15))
 (via (at 89.662 57.912) (size 0.8) (drill 0.4) (layers "F.Cu" "B.Cu") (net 15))
 (segment (start 89.789 57.785) (end 92.116 57.785) (width 0.25) (layer "B.Cu") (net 15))
 (segment (start 89.662 57.912) (end 89.789 57.785) (width 0.25) (layer "B.Cu") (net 15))
 (segment (start 115.189 62.865) (end 115.316 62.738) (width 0.25) (layer "F.Cu") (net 11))
 (segment (start 115.316 62.738) (end 115.316 55.88) (width 0.25) (layer "F.Cu") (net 11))
 (segment (start 109.4975 62.865) (end 115.189 62.865) (width 0.25) (layer "F.Cu") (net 11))
 (segment (start 115.316 55.88) (end 113.5325 55.88) (width 0.25) (layer "F.Cu") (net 11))
 (segment (start 114.808 56.896) (end 114.808 57.912) (width 0.25) (layer "F.Cu") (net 12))
 (segment (start 114.742 56.83) (end 114.808 56.896) (width 0.25) (layer "F.Cu") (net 12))
 (segment (start 114.808 57.912) (end 112.0435 57.912) (width 0.25) (layer "F.Cu") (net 12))
 (segment (start 112.0435 57.912) (end 112.014 57.8825) (width 0.25) (layer "F.Cu") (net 12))
 (segment (start 113.5325 56.83) (end 114.742 56.83) (width 0.25) (layer "F.Cu") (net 12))
 (via (at 112.014 57.8825) (size 0.8) (drill 0.4) (layers "F.Cu" "B.Cu") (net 12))
 (segment (start 109.982 57.649386) (end 109.474 57.141386) (width 0.25) (layer "B.Cu") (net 12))
 (segment (start 109.474 57.141386) (end 109.474 56.896) (width 0.25) (layer "B.Cu") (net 12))
 (segment (start 109.982 57.658) (end 109.982 57.649386) (width 0.25) (layer "B.Cu") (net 12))
 (segment (start 111.7895 57.658) (end 109.982 57.658) (width 0.25) (layer "B.Cu") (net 12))
 (segment (start 112.014 57.8825) (end 111.7895 57.658) (width 0.25) (layer "B.Cu") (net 12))
 (segment (start 109.474 56.896) (end 109.54 56.83) (width 0.25) (layer "B.Cu") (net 12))
 (segment (start 109.54 56.83) (end 110.6225 56.83) (width 0.25) (layer "B.Cu") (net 12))
 (segment (start 113.538 53.086) (end 108.966 53.086) (width 0.25) (layer "F.Cu") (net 13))
 (segment (start 113.5325 54.93) (end 113.5325 53.0915) (width 0.25) (layer "F.Cu") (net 13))
 (segment (start 108.966 53.086) (end 108.966 54.864) (width 0.25) (layer "F.Cu") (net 13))
 (segment (start 113.5325 53.0915) (end 113.538 53.086) (width 0.25) (layer "F.Cu") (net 13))
 (via (at 108.966 54.864) (size 0.8) (drill 0.4) (layers "F.Cu" "B.Cu") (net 13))
 (segment (start 110.5565 54.864) (end 110.6225 54.93) (width 0.25) (layer "B.Cu") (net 13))
 (segment (start 108.966 54.864) (end 110.5565 54.864) (width 0.25) (layer "B.Cu") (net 13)))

